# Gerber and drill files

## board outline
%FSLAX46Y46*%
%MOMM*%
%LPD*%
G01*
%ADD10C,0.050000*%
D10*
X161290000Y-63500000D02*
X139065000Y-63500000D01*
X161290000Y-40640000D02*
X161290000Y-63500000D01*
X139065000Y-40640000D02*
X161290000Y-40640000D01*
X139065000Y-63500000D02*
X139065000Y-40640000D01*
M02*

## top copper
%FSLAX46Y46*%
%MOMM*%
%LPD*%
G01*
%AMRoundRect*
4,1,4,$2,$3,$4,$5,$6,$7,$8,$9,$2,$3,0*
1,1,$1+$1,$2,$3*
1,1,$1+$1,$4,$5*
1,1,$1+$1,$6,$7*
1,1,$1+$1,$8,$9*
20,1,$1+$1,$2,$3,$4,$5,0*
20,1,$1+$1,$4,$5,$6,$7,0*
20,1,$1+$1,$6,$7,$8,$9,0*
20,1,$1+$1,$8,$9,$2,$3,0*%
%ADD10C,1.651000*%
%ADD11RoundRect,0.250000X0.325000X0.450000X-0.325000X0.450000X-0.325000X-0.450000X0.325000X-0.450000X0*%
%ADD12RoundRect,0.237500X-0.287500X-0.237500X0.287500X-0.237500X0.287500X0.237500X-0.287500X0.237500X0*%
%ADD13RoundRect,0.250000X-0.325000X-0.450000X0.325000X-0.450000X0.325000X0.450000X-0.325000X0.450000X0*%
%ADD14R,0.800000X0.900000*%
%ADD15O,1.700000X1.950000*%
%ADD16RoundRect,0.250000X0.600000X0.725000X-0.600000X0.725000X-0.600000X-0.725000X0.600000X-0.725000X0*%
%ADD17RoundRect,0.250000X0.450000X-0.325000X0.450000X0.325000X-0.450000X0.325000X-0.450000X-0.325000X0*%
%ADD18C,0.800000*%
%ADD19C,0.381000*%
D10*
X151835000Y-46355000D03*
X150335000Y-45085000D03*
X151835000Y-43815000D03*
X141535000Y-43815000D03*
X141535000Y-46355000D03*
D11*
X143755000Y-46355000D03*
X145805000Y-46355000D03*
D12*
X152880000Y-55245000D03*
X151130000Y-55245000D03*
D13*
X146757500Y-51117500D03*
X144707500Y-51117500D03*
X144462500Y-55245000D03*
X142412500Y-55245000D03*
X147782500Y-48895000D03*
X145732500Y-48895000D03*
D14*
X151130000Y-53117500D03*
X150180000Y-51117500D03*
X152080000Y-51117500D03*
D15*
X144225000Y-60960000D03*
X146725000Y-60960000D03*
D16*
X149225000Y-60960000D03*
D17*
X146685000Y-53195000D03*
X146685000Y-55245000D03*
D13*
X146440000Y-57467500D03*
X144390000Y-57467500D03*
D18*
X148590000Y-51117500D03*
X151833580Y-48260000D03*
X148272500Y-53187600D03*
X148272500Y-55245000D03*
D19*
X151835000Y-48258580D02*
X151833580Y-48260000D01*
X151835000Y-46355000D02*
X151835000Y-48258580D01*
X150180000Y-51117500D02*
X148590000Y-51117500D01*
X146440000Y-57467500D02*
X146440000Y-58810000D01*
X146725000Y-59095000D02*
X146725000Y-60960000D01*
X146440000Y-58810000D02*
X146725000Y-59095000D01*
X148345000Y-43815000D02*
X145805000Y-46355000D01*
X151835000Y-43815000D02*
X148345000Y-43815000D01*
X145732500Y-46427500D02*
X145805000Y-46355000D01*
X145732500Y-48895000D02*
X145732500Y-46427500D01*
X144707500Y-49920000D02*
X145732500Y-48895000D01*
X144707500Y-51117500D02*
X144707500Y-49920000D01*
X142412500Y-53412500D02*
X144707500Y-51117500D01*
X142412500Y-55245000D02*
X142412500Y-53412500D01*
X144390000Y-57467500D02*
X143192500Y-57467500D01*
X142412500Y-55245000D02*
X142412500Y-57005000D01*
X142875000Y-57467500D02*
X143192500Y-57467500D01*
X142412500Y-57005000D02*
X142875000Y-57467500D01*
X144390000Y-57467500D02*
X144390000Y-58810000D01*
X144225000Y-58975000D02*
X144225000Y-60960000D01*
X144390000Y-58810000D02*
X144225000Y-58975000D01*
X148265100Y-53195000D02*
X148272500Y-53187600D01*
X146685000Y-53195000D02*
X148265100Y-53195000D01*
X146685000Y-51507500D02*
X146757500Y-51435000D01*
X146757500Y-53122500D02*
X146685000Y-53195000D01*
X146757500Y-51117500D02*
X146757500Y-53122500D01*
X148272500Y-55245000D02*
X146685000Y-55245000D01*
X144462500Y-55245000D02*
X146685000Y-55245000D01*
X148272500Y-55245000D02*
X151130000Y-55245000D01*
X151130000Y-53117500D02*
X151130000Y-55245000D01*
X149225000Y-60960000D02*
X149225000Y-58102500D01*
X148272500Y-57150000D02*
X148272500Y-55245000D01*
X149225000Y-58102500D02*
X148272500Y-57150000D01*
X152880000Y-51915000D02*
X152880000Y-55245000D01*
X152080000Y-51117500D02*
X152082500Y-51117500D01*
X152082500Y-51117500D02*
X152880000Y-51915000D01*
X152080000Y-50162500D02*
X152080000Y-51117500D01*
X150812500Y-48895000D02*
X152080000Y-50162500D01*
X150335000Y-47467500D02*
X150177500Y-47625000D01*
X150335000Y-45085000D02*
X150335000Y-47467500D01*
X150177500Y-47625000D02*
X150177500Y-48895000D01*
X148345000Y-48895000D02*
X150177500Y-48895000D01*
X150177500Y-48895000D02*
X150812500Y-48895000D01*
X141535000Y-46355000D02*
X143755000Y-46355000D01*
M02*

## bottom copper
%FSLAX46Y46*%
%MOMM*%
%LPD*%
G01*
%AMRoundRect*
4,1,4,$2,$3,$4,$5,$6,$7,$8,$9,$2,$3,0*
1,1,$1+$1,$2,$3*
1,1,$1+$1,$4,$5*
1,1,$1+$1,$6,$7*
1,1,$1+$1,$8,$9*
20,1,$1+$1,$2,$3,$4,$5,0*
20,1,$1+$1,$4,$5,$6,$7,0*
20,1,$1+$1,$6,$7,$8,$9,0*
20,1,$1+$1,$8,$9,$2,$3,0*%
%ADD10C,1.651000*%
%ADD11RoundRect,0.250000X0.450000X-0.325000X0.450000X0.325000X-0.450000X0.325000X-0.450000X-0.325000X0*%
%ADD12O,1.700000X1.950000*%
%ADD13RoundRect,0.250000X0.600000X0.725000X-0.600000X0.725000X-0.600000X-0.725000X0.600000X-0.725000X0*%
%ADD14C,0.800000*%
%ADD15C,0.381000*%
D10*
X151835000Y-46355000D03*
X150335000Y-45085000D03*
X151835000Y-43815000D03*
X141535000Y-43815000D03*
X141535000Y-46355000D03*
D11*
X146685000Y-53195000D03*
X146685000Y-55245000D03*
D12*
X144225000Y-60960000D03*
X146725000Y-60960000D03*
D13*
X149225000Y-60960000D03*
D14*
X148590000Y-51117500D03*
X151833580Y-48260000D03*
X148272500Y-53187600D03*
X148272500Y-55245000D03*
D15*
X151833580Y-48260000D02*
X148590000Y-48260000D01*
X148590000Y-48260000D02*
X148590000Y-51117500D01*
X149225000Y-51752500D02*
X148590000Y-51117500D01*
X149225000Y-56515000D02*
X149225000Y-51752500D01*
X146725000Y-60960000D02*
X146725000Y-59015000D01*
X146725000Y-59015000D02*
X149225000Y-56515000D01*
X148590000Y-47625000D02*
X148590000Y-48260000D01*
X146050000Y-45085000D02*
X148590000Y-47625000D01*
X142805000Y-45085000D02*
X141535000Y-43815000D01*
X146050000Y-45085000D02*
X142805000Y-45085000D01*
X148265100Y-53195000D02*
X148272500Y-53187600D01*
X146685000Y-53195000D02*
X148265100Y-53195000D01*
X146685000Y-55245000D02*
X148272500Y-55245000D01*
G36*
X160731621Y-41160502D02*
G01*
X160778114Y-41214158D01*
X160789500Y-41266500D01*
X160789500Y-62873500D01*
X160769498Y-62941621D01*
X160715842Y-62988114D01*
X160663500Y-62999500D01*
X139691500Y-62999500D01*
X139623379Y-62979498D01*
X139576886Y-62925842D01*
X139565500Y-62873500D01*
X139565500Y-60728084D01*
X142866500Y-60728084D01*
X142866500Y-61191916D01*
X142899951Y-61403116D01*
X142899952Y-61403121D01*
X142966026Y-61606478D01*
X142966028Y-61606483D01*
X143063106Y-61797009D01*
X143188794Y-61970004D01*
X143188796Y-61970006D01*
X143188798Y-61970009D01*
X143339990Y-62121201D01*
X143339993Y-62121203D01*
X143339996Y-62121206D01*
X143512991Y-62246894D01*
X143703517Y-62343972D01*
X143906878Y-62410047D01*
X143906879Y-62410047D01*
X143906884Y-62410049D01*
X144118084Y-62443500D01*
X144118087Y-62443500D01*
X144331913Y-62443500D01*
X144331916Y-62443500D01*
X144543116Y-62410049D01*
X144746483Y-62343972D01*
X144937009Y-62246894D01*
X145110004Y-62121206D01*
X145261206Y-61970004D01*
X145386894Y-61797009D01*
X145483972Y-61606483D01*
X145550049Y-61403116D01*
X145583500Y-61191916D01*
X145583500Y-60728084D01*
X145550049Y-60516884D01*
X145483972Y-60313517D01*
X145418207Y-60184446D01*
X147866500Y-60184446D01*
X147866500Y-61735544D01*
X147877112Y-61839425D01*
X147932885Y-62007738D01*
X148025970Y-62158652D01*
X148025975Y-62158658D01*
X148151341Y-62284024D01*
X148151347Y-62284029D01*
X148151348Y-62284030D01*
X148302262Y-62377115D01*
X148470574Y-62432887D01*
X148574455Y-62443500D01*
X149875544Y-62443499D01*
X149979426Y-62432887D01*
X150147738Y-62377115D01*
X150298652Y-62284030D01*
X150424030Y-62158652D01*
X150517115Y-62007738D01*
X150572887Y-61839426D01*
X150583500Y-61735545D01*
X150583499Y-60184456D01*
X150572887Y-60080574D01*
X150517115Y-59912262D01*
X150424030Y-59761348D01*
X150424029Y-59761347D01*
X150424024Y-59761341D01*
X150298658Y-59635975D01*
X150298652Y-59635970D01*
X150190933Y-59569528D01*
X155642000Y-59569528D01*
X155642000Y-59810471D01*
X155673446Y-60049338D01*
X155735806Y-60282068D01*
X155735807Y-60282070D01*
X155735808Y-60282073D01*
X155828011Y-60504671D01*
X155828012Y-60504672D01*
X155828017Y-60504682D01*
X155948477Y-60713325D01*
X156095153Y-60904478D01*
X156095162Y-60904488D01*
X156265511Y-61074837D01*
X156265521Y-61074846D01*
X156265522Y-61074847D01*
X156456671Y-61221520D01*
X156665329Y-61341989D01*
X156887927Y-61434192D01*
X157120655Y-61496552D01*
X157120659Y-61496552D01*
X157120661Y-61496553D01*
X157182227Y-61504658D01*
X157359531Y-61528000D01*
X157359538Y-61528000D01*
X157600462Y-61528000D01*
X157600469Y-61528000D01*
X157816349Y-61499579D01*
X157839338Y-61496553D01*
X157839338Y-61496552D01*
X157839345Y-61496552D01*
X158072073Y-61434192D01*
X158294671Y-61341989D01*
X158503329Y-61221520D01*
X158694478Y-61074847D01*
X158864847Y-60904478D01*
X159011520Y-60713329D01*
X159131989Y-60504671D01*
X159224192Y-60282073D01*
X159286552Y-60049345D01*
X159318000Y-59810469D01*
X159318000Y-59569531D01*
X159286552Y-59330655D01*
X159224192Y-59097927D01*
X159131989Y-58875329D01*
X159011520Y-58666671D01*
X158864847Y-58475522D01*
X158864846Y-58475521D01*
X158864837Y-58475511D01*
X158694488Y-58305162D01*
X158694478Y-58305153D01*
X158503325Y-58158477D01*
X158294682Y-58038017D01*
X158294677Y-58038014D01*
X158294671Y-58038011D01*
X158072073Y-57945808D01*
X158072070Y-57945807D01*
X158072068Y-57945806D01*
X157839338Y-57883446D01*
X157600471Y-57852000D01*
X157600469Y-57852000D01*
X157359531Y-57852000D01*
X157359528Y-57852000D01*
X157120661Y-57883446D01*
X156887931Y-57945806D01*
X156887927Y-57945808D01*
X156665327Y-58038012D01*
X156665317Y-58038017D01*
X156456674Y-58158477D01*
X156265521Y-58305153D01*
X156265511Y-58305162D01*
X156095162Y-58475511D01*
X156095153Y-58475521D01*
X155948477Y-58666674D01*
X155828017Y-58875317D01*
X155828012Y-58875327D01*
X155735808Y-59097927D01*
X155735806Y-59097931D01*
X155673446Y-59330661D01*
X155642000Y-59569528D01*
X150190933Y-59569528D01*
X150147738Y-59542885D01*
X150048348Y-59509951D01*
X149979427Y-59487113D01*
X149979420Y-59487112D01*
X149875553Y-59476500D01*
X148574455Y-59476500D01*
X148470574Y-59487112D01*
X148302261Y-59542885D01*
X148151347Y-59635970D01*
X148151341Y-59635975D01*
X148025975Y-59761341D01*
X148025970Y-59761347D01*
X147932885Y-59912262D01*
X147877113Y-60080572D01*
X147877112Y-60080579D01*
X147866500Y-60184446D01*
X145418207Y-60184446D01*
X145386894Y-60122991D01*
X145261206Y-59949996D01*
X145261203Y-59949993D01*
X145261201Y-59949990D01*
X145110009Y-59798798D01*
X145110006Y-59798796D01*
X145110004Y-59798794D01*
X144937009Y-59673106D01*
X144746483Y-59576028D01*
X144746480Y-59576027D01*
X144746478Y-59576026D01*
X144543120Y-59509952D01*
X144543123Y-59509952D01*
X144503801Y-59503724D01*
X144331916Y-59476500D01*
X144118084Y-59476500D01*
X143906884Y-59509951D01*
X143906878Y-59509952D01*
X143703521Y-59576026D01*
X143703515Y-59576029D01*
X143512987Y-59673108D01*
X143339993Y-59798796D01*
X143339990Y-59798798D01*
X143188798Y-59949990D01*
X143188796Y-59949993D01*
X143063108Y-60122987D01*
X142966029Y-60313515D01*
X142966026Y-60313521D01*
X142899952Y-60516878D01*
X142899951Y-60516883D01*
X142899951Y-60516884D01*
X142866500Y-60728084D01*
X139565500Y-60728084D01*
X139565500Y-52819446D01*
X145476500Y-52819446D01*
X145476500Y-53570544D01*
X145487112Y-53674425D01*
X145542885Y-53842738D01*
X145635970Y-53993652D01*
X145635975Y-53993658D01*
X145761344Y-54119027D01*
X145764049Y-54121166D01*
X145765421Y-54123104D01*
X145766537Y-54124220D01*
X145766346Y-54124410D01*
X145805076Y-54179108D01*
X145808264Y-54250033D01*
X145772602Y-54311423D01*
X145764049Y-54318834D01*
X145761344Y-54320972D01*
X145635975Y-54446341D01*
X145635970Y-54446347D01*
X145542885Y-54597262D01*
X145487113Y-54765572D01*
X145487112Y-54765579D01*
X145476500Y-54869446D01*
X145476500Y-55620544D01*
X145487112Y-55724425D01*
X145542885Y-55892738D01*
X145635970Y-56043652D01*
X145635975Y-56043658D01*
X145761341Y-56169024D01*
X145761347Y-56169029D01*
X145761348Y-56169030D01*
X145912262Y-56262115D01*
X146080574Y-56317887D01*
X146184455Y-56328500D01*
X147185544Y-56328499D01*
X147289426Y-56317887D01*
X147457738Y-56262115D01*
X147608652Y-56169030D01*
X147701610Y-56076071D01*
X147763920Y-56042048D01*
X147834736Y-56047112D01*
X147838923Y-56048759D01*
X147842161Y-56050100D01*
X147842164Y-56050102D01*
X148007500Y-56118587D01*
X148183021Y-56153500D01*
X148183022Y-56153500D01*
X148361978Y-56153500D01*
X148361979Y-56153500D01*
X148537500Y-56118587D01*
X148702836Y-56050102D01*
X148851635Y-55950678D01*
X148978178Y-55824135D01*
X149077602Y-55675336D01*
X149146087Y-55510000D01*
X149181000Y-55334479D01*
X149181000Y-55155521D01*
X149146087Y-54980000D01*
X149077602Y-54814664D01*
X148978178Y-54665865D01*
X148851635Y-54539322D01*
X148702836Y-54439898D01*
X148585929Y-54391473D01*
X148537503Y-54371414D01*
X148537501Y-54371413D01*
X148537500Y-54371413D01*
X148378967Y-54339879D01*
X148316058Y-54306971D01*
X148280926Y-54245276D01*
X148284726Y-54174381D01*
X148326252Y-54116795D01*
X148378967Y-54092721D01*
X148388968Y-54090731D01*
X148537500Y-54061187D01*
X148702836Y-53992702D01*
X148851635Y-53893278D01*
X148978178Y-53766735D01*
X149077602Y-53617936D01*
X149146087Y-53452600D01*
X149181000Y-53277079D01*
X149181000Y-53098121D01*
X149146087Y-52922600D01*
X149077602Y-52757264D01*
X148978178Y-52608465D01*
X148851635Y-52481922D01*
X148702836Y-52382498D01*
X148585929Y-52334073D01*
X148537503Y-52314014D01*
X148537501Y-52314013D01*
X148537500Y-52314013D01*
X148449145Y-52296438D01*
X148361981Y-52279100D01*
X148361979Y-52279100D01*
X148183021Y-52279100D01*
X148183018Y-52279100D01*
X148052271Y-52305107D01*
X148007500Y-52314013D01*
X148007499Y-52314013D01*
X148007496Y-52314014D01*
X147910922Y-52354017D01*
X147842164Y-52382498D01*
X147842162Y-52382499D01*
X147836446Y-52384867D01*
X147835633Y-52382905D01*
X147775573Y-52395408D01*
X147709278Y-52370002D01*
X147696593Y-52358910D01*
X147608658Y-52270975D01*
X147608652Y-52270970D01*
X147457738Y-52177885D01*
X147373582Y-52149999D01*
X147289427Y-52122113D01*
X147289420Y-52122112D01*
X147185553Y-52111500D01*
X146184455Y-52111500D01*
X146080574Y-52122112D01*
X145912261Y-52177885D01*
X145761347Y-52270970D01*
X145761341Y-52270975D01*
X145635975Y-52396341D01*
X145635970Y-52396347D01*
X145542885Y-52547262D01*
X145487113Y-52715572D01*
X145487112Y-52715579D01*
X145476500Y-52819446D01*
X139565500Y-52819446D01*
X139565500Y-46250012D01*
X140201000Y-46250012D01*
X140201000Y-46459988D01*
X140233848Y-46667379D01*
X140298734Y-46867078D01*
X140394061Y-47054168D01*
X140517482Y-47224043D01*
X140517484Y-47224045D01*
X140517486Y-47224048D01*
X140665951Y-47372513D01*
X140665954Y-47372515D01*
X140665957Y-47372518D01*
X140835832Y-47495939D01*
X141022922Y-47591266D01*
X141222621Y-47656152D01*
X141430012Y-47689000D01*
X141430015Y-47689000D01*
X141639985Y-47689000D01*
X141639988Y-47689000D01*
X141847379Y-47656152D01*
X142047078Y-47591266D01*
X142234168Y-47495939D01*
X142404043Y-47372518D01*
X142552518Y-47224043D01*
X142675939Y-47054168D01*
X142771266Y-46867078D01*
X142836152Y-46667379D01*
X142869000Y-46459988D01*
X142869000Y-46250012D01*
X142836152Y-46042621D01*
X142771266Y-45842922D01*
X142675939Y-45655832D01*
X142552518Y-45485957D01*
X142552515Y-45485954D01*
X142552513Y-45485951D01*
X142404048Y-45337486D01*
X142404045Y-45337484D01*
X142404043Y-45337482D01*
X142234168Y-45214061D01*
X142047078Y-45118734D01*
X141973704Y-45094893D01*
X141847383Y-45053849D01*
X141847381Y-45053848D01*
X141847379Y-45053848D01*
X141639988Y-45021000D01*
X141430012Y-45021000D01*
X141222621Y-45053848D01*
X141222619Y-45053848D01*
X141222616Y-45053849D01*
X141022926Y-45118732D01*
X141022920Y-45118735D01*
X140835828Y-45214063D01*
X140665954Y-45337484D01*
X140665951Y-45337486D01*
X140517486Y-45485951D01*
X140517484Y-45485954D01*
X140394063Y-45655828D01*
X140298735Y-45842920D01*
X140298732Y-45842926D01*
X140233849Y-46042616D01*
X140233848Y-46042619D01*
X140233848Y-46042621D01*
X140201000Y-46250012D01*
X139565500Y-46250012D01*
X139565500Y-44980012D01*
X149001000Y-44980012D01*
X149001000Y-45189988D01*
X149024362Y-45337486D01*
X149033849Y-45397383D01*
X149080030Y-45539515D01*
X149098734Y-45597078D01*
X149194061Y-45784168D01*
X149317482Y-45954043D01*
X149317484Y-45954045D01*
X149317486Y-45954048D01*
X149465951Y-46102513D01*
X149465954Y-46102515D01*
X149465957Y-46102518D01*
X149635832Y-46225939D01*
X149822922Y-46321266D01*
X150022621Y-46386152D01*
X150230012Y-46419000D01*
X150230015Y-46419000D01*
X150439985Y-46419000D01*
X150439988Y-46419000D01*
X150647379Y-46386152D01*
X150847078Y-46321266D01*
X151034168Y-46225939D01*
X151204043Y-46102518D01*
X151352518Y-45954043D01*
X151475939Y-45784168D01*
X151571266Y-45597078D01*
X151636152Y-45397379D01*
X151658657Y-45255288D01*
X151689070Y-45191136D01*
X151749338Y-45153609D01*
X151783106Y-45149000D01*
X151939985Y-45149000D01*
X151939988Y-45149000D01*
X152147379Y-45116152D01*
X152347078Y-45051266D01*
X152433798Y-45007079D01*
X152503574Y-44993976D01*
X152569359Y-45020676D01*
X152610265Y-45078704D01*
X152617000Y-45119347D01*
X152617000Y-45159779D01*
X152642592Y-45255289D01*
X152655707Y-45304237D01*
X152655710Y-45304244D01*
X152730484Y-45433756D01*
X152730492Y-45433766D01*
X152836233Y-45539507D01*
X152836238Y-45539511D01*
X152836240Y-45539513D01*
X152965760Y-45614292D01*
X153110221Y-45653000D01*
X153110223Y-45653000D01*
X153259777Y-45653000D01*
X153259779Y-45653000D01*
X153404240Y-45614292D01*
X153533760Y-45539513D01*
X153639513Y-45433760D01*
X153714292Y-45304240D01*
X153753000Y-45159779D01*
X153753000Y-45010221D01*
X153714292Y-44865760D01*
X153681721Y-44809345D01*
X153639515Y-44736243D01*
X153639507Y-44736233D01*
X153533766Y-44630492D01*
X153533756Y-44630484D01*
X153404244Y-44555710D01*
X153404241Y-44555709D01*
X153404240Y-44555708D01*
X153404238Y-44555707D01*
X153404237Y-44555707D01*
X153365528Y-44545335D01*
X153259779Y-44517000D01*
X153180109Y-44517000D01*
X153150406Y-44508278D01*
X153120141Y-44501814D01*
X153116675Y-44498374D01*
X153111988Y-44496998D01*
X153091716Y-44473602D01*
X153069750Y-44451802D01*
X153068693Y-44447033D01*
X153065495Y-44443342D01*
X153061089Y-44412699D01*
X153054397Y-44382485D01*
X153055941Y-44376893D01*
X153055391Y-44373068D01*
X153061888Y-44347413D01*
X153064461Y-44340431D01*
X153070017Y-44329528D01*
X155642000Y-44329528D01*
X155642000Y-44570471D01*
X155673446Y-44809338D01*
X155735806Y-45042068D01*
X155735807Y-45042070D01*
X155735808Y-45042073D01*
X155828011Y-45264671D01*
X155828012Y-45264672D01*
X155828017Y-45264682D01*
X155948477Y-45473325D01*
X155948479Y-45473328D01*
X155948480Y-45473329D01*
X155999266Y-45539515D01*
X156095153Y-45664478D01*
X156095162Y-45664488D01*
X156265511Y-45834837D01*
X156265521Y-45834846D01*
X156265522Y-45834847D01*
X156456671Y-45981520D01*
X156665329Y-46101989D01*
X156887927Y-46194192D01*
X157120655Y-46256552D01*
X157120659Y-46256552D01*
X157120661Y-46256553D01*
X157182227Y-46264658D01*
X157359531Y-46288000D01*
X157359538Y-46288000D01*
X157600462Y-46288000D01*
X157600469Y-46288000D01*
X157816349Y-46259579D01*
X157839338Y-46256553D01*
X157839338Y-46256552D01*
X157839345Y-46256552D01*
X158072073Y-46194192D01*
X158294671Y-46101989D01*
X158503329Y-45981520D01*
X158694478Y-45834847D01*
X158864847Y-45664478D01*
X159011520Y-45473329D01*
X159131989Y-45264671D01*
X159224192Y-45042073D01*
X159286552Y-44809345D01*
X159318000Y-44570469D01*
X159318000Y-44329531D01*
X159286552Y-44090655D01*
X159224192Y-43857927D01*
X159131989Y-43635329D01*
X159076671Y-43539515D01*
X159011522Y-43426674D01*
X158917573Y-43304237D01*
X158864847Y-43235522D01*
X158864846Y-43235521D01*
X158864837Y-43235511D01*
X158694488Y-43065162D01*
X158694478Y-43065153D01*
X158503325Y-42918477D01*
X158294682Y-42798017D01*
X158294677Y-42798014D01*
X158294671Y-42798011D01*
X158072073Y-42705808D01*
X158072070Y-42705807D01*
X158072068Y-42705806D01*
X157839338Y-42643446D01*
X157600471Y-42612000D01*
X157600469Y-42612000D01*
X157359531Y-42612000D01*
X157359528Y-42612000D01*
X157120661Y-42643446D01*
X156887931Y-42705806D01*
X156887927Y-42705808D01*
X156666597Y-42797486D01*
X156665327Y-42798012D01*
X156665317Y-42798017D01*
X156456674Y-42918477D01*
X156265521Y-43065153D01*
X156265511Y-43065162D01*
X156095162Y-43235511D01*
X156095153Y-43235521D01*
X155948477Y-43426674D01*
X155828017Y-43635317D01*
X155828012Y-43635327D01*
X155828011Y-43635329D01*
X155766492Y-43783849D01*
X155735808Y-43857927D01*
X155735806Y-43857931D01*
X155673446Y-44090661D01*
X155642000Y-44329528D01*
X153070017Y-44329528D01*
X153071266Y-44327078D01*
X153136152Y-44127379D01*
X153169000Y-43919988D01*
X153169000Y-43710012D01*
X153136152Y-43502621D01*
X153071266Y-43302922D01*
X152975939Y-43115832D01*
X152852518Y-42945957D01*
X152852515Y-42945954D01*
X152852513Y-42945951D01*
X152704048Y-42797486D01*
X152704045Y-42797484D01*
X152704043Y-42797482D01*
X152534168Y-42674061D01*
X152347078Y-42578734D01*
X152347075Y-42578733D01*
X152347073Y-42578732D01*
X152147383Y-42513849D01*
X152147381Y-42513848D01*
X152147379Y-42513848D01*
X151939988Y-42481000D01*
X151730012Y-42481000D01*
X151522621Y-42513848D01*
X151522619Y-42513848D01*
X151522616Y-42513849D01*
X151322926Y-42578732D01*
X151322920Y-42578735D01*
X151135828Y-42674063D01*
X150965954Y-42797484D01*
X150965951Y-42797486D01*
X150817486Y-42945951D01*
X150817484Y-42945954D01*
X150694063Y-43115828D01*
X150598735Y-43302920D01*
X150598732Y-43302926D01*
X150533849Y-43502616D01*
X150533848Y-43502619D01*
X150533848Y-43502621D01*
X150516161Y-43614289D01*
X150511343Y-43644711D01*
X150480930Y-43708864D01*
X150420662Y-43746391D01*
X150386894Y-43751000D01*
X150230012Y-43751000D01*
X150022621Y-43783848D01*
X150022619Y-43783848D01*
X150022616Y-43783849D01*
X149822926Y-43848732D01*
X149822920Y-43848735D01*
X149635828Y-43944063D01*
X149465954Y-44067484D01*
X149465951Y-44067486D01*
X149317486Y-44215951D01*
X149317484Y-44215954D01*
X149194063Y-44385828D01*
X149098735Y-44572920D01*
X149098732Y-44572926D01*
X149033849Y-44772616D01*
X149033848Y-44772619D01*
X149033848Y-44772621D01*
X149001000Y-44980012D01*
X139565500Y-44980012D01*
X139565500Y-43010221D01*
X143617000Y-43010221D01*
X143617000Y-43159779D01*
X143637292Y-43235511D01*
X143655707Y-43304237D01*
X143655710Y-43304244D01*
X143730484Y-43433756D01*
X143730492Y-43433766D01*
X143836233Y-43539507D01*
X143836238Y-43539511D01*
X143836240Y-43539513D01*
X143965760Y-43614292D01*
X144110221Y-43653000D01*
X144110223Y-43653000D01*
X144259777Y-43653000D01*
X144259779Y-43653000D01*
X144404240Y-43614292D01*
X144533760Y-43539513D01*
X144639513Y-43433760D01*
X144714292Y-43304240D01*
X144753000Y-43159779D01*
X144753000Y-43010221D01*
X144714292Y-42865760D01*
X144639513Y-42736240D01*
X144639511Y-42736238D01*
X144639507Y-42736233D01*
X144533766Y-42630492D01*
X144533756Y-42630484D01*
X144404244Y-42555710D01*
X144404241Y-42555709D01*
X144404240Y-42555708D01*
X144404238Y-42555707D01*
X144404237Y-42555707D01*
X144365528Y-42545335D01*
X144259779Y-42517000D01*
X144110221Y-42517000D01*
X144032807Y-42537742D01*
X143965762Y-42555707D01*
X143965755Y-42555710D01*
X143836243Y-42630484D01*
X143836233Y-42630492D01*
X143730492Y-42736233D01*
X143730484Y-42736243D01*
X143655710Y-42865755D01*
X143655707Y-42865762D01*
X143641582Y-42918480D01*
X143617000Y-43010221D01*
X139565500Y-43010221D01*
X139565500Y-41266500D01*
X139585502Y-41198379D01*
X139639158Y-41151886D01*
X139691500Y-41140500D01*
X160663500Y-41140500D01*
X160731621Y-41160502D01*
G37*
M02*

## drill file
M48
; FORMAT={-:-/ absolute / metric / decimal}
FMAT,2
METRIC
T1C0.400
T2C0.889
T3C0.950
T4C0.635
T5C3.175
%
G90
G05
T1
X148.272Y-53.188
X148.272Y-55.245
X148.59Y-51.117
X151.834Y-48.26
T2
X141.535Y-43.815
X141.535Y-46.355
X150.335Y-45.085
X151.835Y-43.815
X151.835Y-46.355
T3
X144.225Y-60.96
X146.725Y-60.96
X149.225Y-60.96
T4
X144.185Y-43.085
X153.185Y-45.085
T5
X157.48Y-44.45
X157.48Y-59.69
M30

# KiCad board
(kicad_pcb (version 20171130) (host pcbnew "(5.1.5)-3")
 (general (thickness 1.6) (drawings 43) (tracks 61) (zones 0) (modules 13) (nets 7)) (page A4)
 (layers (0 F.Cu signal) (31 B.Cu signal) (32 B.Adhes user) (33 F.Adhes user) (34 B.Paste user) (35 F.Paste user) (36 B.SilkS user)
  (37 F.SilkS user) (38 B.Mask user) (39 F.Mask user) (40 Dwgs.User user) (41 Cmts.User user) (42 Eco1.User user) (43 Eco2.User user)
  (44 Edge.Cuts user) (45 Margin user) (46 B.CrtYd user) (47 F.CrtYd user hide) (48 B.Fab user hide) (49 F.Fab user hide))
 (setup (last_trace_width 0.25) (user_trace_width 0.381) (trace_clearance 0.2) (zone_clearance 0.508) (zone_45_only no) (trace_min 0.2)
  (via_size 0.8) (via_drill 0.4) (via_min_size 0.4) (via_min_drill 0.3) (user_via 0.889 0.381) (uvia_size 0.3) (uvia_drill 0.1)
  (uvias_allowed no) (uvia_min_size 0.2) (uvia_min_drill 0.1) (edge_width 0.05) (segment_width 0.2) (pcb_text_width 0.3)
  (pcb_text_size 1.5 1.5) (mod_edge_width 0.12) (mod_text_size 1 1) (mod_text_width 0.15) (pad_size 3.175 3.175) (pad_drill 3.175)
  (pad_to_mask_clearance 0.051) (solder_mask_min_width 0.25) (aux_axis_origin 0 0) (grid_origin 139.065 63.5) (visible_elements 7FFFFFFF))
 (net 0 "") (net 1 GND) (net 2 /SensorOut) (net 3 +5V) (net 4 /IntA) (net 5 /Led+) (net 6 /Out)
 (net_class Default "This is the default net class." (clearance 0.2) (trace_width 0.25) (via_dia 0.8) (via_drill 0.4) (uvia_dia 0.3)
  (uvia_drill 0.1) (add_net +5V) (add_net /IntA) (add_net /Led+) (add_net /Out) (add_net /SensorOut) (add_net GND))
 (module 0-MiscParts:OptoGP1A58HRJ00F (layer B.Cu) (at 146.685 45.085 180)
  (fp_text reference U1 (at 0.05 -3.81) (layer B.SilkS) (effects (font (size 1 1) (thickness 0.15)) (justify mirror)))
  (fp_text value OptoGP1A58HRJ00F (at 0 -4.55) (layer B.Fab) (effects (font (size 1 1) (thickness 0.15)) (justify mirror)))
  (pad "" np_thru_hole circle (at 2.5 2 180) (size 0.635 0.635) (drill 0.635) (layers *.Cu *.Mask))
  (pad "" np_thru_hole circle (at -6.5 0 180) (size 0.635 0.635) (drill 0.635) (layers *.Cu *.Mask))
  (pad 5 thru_hole circle (at -5.15 -1.27 180) (size 1.651 1.651) (drill 0.889) (layers *.Cu *.Mask) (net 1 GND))
  (pad 4 thru_hole circle (at -3.65 0 180) (size 1.651 1.651) (drill 0.889) (layers *.Cu *.Mask) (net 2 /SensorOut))
  (pad 3 thru_hole circle (at -5.15 1.27 180) (size 1.651 1.651) (drill 0.889) (layers *.Cu *.Mask) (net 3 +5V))
  (pad 2 thru_hole circle (at 5.15 1.27 180) (size 1.651 1.651) (drill 0.889) (layers *.Cu *.Mask) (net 1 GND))
  (pad 1 thru_hole circle (at 5.15 -1.27 180) (size 1.651 1.651) (drill 0.889) (layers *.Cu *.Mask) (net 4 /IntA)))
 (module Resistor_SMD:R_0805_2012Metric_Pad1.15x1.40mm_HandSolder (layer F.Cu) (at 144.78 46.355 180)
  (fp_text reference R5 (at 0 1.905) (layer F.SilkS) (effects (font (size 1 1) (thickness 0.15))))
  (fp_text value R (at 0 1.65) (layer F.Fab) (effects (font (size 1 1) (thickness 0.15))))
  (pad 2 smd roundrect (at 1.025 0 180) (size 1.15 1.4) (layers F.Cu F.Paste F.Mask) (roundrect_rratio 0.217391) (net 4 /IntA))
  (pad 1 smd roundrect (at -1.025 0 180) (size 1.15 1.4) (layers F.Cu F.Paste F.Mask) (roundrect_rratio 0.217391) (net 3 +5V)))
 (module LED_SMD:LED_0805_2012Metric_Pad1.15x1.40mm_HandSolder (layer B.Cu) (at 146.685 54.22 90)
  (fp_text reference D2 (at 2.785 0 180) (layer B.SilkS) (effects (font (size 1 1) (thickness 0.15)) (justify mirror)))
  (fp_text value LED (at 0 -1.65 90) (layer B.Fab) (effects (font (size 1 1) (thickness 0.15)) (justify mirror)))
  (pad 2 smd roundrect (at 1.025 0 90) (size 1.15 1.4) (layers B.Cu B.Paste B.Mask) (roundrect_rratio 0.217391) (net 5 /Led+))
  (pad 1 smd roundrect (at -1.025 0 90) (size 1.15 1.4) (layers B.Cu B.Paste B.Mask) (roundrect_rratio 0.217391) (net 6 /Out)))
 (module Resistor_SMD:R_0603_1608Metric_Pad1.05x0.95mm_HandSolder (layer F.Cu) (at 152.005 55.245)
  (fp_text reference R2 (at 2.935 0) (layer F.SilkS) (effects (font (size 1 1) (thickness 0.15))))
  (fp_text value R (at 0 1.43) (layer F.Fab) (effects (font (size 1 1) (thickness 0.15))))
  (pad 2 smd roundrect (at 0.875 0) (size 1.05 0.95) (layers F.Cu F.Paste F.Mask) (roundrect_rratio 0.25) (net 2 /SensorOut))
  (pad 1 smd roundrect (at -0.875 0) (size 1.05 0.95) (layers F.Cu F.Paste F.Mask) (roundrect_rratio 0.25) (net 6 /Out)))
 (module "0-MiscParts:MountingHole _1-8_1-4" (layer F.Cu) (at 157.48 44.45)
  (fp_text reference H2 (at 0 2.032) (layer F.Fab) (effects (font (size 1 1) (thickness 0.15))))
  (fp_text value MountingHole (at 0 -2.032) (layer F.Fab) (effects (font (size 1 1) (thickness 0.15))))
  (pad "" np_thru_hole circle (at 0 0) (size 3.175 3.175) (drill 3.175) (layers *.Cu *.Mask)))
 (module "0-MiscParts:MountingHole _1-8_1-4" (layer F.Cu) (at 157.48 59.69)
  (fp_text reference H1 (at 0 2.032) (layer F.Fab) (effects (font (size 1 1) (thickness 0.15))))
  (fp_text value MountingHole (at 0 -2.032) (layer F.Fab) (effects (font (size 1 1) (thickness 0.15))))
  (pad "" np_thru_hole circle (at 0 0) (size 3.175 3.175) (drill 3.175) (layers *.Cu *.Mask)))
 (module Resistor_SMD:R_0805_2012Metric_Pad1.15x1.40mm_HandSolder (layer F.Cu) (at 145.7325 51.1175)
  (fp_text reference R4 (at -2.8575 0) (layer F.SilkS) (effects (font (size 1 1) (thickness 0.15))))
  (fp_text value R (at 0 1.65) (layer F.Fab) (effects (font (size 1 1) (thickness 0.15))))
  (pad 2 smd roundrect (at 1.025 0) (size 1.15 1.4) (layers F.Cu F.Paste F.Mask) (roundrect_rratio 0.217391) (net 5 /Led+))
  (pad 1 smd roundrect (at -1.025 0) (size 1.15 1.4) (layers F.Cu F.Paste F.Mask) (roundrect_rratio 0.217391) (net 3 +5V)))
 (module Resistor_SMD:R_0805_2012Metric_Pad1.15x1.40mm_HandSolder (layer F.Cu) (at 143.4375 55.245)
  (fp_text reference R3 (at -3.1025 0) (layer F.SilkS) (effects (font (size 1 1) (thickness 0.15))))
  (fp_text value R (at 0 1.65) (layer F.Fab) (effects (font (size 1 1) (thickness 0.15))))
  (pad 2 smd roundrect (at 1.025 0) (size 1.15 1.4) (layers F.Cu F.Paste F.Mask) (roundrect_rratio 0.217391) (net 6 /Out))
  (pad 1 smd roundrect (at -1.025 0) (size 1.15 1.4) (layers F.Cu F.Paste F.Mask) (roundrect_rratio 0.217391) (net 3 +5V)))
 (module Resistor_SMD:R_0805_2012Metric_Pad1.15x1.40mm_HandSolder (layer F.Cu) (at 146.7575 48.895)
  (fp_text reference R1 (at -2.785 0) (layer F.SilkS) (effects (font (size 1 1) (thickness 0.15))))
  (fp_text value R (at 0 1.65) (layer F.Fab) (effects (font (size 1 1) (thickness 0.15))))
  (pad 2 smd roundrect (at 1.025 0) (size 1.15 1.4) (layers F.Cu F.Paste F.Mask) (roundrect_rratio 0.217391) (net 2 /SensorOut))
  (pad 1 smd roundrect (at -1.025 0) (size 1.15 1.4) (layers F.Cu F.Paste F.Mask) (roundrect_rratio 0.217391) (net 3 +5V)))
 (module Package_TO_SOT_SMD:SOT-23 (layer F.Cu) (at 151.13 52.1175 270)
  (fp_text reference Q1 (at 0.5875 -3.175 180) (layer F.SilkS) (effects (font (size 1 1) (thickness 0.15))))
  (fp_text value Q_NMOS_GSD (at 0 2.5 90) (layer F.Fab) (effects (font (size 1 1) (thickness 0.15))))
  (pad 3 smd rect (at 1 0 270) (size 0.9 0.8) (layers F.Cu F.Paste F.Mask) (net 6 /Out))
  (pad 2 smd rect (at -1 0.95 270) (size 0.9 0.8) (layers F.Cu F.Paste F.Mask) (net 1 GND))
  (pad 1 smd rect (at -1 -0.95 270) (size 0.9 0.8) (layers F.Cu F.Paste F.Mask) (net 2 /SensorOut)))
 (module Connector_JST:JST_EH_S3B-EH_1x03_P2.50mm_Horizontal (layer F.Cu) (at 149.225 60.96 180)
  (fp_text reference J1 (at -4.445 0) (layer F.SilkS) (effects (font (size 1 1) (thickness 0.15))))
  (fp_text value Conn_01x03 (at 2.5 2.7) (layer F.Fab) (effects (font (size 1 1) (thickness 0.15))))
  (pad 3 thru_hole oval (at 5 0 180) (size 1.7 1.95) (drill 0.95) (layers *.Cu *.Mask) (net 3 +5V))
  (pad 2 thru_hole oval (at 2.5 0 180) (size 1.7 1.95) (drill 0.95) (layers *.Cu *.Mask) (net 1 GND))
  (pad 1 thru_hole roundrect (at 0 0 180) (size 1.7 1.95) (drill 0.95) (layers *.Cu *.Mask) (roundrect_rratio 0.147059) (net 6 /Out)))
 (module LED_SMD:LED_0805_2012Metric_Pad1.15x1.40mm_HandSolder (layer F.Cu) (at 146.685 54.22 90)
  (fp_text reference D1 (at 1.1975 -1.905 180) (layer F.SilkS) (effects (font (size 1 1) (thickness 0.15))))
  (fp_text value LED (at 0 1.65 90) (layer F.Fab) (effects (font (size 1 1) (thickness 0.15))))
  (pad 2 smd roundrect (at 1.025 0 90) (size 1.15 1.4) (layers F.Cu F.Paste F.Mask) (roundrect_rratio 0.217391) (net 5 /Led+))
  (pad 1 smd roundrect (at -1.025 0 90) (size 1.15 1.4) (layers F.Cu F.Paste F.Mask) (roundrect_rratio 0.217391) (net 6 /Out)))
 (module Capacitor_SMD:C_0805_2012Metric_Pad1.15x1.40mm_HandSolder (layer F.Cu) (at 145.415 57.4675)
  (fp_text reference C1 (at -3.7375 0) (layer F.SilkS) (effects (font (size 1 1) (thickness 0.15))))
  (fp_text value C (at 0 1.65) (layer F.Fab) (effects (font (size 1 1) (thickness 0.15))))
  (pad 2 smd roundrect (at 1.025 0) (size 1.15 1.4) (layers F.Cu F.Paste F.Mask) (roundrect_rratio 0.217391) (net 1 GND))
  (pad 1 smd roundrect (at -1.025 0) (size 1.15 1.4) (layers F.Cu F.Paste F.Mask) (roundrect_rratio 0.217391) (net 3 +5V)))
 (gr_line (start 161.29 63.5) (end 139.065 63.5) (layer Edge.Cuts) (width 0.05))
 (gr_line (start 161.29 40.64) (end 161.29 63.5) (layer Edge.Cuts) (width 0.05))
 (gr_line (start 139.065 40.64) (end 161.29 40.64) (layer Edge.Cuts) (width 0.05))
 (gr_line (start 139.065 63.5) (end 139.065 40.64) (layer Edge.Cuts) (width 0.05))
 (via (at 148.59 51.1175) (size 0.8) (drill 0.4) (layers F.Cu B.Cu) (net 1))
 (via (at 151.83358 48.26) (size 0.8) (drill 0.4) (layers F.Cu B.Cu) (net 1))
 (segment (start 151.835 48.25858) (end 151.83358 48.26) (width 0.381) (layer F.Cu) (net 1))
 (segment (start 151.835 46.355) (end 151.835 48.25858) (width 0.381) (layer F.Cu) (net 1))
 (segment (start 150.18 51.1175) (end 148.59 51.1175) (width 0.381) (layer F.Cu) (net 1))
 (segment (start 151.83358 48.26) (end 148.59 48.26) (width 0.381) (layer B.Cu) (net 1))
 (segment (start 148.59 48.26) (end 148.59 51.1175) (width 0.381) (layer B.Cu) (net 1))
 (segment (start 149.225 51.7525) (end 148.59 51.1175) (width 0.381) (layer B.Cu) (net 1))
 (segment (start 149.225 56.515) (end 149.225 51.7525) (width 0.381) (layer B.Cu) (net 1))
 (segment (start 146.725 60.96) (end 146.725 59.015) (width 0.381) (layer B.Cu) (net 1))
 (segment (start 146.725 59.015) (end 149.225 56.515) (width 0.381) (layer B.Cu) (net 1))
 (segment (start 146.44 57.4675) (end 146.44 58.81) (width 0.381) (layer F.Cu) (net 1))
 (segment (start 146.725 59.095) (end 146.725 60.96) (width 0.381) (layer F.Cu) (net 1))
 (segment (start 146.44 58.81) (end 146.725 59.095) (width 0.381) (layer F.Cu) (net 1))
 (segment (start 148.59 47.625) (end 148.59 48.26) (width 0.381) (layer B.Cu) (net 1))
 (segment (start 146.05 45.085) (end 148.59 47.625) (width 0.381) (layer B.Cu) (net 1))
 (segment (start 142.805 45.085) (end 141.535 43.815) (width 0.381) (layer B.Cu) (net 1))
 (segment (start 146.05 45.085) (end 142.805 45.085) (width 0.381) (layer B.Cu) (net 1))
 (segment (start 148.345 43.815) (end 145.805 46.355) (width 0.381) (layer F.Cu) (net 3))
 (segment (start 151.835 43.815) (end 148.345 43.815) (width 0.381) (layer F.Cu) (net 3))
 (segment (start 145.7325 46.4275) (end 145.805 46.355) (width 0.381) (layer F.Cu) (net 3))
 (segment (start 145.7325 48.895) (end 145.7325 46.4275) (width 0.381) (layer F.Cu) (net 3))
 (segment (start 144.7075 49.92) (end 145.7325 48.895) (width 0.381) (layer F.Cu) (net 3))
 (segment (start 144.7075 51.1175) (end 144.7075 49.92) (width 0.381) (layer F.Cu) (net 3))
 (segment (start 142.4125 53.4125) (end 144.7075 51.1175) (width 0.381) (layer F.Cu) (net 3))
 (segment (start 142.4125 55.245) (end 142.4125 53.4125) (width 0.381) (layer F.Cu) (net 3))
 (segment (start 144.39 57.4675) (end 143.1925 57.4675) (width 0.381) (layer F.Cu) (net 3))
 (segment (start 142.4125 55.245) (end 142.4125 57.005) (width 0.381) (layer F.Cu) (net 3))
 (segment (start 142.875 57.4675) (end 143.1925 57.4675) (width 0.381) (layer F.Cu) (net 3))
 (segment (start 142.4125 57.005) (end 142.875 57.4675) (width 0.381) (layer F.Cu) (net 3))
 (segment (start 144.39 57.4675) (end 144.39 58.81) (width 0.381) (layer F.Cu) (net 3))
 (segment (start 144.225 58.975) (end 144.225 60.96) (width 0.381) (layer F.Cu) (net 3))
 (segment (start 144.39 58.81) (end 144.225 58.975) (width 0.381) (layer F.Cu) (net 3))
 (via (at 148.2725 53.1876) (size 0.8) (drill 0.4) (layers F.Cu B.Cu) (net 5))
 (segment (start 148.2651 53.195) (end 148.2725 53.1876) (width 0.381) (layer F.Cu) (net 5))
 (segment (start 146.685 53.195) (end 148.2651 53.195) (width 0.381) (layer F.Cu) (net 5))
 (segment (start 148.2651 53.195) (end 148.2725 53.1876) (width 0.381) (layer B.Cu) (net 5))
 (segment (start 146.685 53.195) (end 148.2651 53.195) (width 0.381) (layer B.Cu) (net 5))
 (segment (start 146.685 51.5075) (end 146.7575 51.435) (width 0.381) (layer F.Cu) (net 5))
 (segment (start 146.7575 53.1225) (end 146.685 53.195) (width 0.381) (layer F.Cu) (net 5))
 (segment (start 146.7575 51.1175) (end 146.7575 53.1225) (width 0.381) (layer F.Cu) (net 5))
 (via (at 148.2725 55.245) (size 0.8) (drill 0.4) (layers F.Cu B.Cu) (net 6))
 (segment (start 148.2725 55.245) (end 146.685 55.245) (width 0.381) (layer F.Cu) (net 6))
 (segment (start 146.685 55.245) (end 148.2725 55.245) (width 0.381) (layer B.Cu) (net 6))
 (segment (start 144.4625 55.245) (end 146.685 55.245) (width 0.381) (layer F.Cu) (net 6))
 (segment (start 148.2725 55.245) (end 151.13 55.245) (width 0.381) (layer F.Cu) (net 6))
 (segment (start 151.13 53.1175) (end 151.13 55.245) (width 0.381) (layer F.Cu) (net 6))
 (segment (start 149.225 60.96) (end 149.225 58.1025) (width 0.381) (layer F.Cu) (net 6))
 (segment (start 148.2725 57.15) (end 148.2725 55.245) (width 0.381) (layer F.Cu) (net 6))
 (segment (start 149.225 58.1025) (end 148.2725 57.15) (width 0.381) (layer F.Cu) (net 6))
 (segment (start 152.88 51.915) (end 152.88 55.245) (width 0.381) (layer F.Cu) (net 2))
 (segment (start 152.08 51.1175) (end 152.0825 51.1175) (width 0.381) (layer F.Cu) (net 2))
 (segment (start 152.0825 51.1175) (end 152.88 51.915) (width 0.381) (layer F.Cu) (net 2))
 (segment (start 152.08 50.1625) (end 152.08 51.1175) (width 0.381) (layer F.Cu) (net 2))
 (segment (start 150.8125 48.895) (end 152.08 50.1625) (width 0.381) (layer F.Cu) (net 2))
 (segment (start 150.335 47.4675) (end 150.1775 47.625) (width 0.381) (layer F.Cu) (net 2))
 (segment (start 150.335 45.085) (end 150.335 47.4675) (width 0.381) (layer F.Cu) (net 2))
 (segment (start 150.1775 47.625) (end 150.1775 48.895) (width 0.381) (layer F.Cu) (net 2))
 (segment (start 148.345 48.895) (end 150.1775 48.895) (width 0.381) (layer F.Cu) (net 2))
 (segment (start 150.1775 48.895) (end 150.8125 48.895) (width 0.381) (layer F.Cu) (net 2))
 (segment (start 141.535 46.355) (end 143.755 46.355) (width 0.381) (layer F.Cu) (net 4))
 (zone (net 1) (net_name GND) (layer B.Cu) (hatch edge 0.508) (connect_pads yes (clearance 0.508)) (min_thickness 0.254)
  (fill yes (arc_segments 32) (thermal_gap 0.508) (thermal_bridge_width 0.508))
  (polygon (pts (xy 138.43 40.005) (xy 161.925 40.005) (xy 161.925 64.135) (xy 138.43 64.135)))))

